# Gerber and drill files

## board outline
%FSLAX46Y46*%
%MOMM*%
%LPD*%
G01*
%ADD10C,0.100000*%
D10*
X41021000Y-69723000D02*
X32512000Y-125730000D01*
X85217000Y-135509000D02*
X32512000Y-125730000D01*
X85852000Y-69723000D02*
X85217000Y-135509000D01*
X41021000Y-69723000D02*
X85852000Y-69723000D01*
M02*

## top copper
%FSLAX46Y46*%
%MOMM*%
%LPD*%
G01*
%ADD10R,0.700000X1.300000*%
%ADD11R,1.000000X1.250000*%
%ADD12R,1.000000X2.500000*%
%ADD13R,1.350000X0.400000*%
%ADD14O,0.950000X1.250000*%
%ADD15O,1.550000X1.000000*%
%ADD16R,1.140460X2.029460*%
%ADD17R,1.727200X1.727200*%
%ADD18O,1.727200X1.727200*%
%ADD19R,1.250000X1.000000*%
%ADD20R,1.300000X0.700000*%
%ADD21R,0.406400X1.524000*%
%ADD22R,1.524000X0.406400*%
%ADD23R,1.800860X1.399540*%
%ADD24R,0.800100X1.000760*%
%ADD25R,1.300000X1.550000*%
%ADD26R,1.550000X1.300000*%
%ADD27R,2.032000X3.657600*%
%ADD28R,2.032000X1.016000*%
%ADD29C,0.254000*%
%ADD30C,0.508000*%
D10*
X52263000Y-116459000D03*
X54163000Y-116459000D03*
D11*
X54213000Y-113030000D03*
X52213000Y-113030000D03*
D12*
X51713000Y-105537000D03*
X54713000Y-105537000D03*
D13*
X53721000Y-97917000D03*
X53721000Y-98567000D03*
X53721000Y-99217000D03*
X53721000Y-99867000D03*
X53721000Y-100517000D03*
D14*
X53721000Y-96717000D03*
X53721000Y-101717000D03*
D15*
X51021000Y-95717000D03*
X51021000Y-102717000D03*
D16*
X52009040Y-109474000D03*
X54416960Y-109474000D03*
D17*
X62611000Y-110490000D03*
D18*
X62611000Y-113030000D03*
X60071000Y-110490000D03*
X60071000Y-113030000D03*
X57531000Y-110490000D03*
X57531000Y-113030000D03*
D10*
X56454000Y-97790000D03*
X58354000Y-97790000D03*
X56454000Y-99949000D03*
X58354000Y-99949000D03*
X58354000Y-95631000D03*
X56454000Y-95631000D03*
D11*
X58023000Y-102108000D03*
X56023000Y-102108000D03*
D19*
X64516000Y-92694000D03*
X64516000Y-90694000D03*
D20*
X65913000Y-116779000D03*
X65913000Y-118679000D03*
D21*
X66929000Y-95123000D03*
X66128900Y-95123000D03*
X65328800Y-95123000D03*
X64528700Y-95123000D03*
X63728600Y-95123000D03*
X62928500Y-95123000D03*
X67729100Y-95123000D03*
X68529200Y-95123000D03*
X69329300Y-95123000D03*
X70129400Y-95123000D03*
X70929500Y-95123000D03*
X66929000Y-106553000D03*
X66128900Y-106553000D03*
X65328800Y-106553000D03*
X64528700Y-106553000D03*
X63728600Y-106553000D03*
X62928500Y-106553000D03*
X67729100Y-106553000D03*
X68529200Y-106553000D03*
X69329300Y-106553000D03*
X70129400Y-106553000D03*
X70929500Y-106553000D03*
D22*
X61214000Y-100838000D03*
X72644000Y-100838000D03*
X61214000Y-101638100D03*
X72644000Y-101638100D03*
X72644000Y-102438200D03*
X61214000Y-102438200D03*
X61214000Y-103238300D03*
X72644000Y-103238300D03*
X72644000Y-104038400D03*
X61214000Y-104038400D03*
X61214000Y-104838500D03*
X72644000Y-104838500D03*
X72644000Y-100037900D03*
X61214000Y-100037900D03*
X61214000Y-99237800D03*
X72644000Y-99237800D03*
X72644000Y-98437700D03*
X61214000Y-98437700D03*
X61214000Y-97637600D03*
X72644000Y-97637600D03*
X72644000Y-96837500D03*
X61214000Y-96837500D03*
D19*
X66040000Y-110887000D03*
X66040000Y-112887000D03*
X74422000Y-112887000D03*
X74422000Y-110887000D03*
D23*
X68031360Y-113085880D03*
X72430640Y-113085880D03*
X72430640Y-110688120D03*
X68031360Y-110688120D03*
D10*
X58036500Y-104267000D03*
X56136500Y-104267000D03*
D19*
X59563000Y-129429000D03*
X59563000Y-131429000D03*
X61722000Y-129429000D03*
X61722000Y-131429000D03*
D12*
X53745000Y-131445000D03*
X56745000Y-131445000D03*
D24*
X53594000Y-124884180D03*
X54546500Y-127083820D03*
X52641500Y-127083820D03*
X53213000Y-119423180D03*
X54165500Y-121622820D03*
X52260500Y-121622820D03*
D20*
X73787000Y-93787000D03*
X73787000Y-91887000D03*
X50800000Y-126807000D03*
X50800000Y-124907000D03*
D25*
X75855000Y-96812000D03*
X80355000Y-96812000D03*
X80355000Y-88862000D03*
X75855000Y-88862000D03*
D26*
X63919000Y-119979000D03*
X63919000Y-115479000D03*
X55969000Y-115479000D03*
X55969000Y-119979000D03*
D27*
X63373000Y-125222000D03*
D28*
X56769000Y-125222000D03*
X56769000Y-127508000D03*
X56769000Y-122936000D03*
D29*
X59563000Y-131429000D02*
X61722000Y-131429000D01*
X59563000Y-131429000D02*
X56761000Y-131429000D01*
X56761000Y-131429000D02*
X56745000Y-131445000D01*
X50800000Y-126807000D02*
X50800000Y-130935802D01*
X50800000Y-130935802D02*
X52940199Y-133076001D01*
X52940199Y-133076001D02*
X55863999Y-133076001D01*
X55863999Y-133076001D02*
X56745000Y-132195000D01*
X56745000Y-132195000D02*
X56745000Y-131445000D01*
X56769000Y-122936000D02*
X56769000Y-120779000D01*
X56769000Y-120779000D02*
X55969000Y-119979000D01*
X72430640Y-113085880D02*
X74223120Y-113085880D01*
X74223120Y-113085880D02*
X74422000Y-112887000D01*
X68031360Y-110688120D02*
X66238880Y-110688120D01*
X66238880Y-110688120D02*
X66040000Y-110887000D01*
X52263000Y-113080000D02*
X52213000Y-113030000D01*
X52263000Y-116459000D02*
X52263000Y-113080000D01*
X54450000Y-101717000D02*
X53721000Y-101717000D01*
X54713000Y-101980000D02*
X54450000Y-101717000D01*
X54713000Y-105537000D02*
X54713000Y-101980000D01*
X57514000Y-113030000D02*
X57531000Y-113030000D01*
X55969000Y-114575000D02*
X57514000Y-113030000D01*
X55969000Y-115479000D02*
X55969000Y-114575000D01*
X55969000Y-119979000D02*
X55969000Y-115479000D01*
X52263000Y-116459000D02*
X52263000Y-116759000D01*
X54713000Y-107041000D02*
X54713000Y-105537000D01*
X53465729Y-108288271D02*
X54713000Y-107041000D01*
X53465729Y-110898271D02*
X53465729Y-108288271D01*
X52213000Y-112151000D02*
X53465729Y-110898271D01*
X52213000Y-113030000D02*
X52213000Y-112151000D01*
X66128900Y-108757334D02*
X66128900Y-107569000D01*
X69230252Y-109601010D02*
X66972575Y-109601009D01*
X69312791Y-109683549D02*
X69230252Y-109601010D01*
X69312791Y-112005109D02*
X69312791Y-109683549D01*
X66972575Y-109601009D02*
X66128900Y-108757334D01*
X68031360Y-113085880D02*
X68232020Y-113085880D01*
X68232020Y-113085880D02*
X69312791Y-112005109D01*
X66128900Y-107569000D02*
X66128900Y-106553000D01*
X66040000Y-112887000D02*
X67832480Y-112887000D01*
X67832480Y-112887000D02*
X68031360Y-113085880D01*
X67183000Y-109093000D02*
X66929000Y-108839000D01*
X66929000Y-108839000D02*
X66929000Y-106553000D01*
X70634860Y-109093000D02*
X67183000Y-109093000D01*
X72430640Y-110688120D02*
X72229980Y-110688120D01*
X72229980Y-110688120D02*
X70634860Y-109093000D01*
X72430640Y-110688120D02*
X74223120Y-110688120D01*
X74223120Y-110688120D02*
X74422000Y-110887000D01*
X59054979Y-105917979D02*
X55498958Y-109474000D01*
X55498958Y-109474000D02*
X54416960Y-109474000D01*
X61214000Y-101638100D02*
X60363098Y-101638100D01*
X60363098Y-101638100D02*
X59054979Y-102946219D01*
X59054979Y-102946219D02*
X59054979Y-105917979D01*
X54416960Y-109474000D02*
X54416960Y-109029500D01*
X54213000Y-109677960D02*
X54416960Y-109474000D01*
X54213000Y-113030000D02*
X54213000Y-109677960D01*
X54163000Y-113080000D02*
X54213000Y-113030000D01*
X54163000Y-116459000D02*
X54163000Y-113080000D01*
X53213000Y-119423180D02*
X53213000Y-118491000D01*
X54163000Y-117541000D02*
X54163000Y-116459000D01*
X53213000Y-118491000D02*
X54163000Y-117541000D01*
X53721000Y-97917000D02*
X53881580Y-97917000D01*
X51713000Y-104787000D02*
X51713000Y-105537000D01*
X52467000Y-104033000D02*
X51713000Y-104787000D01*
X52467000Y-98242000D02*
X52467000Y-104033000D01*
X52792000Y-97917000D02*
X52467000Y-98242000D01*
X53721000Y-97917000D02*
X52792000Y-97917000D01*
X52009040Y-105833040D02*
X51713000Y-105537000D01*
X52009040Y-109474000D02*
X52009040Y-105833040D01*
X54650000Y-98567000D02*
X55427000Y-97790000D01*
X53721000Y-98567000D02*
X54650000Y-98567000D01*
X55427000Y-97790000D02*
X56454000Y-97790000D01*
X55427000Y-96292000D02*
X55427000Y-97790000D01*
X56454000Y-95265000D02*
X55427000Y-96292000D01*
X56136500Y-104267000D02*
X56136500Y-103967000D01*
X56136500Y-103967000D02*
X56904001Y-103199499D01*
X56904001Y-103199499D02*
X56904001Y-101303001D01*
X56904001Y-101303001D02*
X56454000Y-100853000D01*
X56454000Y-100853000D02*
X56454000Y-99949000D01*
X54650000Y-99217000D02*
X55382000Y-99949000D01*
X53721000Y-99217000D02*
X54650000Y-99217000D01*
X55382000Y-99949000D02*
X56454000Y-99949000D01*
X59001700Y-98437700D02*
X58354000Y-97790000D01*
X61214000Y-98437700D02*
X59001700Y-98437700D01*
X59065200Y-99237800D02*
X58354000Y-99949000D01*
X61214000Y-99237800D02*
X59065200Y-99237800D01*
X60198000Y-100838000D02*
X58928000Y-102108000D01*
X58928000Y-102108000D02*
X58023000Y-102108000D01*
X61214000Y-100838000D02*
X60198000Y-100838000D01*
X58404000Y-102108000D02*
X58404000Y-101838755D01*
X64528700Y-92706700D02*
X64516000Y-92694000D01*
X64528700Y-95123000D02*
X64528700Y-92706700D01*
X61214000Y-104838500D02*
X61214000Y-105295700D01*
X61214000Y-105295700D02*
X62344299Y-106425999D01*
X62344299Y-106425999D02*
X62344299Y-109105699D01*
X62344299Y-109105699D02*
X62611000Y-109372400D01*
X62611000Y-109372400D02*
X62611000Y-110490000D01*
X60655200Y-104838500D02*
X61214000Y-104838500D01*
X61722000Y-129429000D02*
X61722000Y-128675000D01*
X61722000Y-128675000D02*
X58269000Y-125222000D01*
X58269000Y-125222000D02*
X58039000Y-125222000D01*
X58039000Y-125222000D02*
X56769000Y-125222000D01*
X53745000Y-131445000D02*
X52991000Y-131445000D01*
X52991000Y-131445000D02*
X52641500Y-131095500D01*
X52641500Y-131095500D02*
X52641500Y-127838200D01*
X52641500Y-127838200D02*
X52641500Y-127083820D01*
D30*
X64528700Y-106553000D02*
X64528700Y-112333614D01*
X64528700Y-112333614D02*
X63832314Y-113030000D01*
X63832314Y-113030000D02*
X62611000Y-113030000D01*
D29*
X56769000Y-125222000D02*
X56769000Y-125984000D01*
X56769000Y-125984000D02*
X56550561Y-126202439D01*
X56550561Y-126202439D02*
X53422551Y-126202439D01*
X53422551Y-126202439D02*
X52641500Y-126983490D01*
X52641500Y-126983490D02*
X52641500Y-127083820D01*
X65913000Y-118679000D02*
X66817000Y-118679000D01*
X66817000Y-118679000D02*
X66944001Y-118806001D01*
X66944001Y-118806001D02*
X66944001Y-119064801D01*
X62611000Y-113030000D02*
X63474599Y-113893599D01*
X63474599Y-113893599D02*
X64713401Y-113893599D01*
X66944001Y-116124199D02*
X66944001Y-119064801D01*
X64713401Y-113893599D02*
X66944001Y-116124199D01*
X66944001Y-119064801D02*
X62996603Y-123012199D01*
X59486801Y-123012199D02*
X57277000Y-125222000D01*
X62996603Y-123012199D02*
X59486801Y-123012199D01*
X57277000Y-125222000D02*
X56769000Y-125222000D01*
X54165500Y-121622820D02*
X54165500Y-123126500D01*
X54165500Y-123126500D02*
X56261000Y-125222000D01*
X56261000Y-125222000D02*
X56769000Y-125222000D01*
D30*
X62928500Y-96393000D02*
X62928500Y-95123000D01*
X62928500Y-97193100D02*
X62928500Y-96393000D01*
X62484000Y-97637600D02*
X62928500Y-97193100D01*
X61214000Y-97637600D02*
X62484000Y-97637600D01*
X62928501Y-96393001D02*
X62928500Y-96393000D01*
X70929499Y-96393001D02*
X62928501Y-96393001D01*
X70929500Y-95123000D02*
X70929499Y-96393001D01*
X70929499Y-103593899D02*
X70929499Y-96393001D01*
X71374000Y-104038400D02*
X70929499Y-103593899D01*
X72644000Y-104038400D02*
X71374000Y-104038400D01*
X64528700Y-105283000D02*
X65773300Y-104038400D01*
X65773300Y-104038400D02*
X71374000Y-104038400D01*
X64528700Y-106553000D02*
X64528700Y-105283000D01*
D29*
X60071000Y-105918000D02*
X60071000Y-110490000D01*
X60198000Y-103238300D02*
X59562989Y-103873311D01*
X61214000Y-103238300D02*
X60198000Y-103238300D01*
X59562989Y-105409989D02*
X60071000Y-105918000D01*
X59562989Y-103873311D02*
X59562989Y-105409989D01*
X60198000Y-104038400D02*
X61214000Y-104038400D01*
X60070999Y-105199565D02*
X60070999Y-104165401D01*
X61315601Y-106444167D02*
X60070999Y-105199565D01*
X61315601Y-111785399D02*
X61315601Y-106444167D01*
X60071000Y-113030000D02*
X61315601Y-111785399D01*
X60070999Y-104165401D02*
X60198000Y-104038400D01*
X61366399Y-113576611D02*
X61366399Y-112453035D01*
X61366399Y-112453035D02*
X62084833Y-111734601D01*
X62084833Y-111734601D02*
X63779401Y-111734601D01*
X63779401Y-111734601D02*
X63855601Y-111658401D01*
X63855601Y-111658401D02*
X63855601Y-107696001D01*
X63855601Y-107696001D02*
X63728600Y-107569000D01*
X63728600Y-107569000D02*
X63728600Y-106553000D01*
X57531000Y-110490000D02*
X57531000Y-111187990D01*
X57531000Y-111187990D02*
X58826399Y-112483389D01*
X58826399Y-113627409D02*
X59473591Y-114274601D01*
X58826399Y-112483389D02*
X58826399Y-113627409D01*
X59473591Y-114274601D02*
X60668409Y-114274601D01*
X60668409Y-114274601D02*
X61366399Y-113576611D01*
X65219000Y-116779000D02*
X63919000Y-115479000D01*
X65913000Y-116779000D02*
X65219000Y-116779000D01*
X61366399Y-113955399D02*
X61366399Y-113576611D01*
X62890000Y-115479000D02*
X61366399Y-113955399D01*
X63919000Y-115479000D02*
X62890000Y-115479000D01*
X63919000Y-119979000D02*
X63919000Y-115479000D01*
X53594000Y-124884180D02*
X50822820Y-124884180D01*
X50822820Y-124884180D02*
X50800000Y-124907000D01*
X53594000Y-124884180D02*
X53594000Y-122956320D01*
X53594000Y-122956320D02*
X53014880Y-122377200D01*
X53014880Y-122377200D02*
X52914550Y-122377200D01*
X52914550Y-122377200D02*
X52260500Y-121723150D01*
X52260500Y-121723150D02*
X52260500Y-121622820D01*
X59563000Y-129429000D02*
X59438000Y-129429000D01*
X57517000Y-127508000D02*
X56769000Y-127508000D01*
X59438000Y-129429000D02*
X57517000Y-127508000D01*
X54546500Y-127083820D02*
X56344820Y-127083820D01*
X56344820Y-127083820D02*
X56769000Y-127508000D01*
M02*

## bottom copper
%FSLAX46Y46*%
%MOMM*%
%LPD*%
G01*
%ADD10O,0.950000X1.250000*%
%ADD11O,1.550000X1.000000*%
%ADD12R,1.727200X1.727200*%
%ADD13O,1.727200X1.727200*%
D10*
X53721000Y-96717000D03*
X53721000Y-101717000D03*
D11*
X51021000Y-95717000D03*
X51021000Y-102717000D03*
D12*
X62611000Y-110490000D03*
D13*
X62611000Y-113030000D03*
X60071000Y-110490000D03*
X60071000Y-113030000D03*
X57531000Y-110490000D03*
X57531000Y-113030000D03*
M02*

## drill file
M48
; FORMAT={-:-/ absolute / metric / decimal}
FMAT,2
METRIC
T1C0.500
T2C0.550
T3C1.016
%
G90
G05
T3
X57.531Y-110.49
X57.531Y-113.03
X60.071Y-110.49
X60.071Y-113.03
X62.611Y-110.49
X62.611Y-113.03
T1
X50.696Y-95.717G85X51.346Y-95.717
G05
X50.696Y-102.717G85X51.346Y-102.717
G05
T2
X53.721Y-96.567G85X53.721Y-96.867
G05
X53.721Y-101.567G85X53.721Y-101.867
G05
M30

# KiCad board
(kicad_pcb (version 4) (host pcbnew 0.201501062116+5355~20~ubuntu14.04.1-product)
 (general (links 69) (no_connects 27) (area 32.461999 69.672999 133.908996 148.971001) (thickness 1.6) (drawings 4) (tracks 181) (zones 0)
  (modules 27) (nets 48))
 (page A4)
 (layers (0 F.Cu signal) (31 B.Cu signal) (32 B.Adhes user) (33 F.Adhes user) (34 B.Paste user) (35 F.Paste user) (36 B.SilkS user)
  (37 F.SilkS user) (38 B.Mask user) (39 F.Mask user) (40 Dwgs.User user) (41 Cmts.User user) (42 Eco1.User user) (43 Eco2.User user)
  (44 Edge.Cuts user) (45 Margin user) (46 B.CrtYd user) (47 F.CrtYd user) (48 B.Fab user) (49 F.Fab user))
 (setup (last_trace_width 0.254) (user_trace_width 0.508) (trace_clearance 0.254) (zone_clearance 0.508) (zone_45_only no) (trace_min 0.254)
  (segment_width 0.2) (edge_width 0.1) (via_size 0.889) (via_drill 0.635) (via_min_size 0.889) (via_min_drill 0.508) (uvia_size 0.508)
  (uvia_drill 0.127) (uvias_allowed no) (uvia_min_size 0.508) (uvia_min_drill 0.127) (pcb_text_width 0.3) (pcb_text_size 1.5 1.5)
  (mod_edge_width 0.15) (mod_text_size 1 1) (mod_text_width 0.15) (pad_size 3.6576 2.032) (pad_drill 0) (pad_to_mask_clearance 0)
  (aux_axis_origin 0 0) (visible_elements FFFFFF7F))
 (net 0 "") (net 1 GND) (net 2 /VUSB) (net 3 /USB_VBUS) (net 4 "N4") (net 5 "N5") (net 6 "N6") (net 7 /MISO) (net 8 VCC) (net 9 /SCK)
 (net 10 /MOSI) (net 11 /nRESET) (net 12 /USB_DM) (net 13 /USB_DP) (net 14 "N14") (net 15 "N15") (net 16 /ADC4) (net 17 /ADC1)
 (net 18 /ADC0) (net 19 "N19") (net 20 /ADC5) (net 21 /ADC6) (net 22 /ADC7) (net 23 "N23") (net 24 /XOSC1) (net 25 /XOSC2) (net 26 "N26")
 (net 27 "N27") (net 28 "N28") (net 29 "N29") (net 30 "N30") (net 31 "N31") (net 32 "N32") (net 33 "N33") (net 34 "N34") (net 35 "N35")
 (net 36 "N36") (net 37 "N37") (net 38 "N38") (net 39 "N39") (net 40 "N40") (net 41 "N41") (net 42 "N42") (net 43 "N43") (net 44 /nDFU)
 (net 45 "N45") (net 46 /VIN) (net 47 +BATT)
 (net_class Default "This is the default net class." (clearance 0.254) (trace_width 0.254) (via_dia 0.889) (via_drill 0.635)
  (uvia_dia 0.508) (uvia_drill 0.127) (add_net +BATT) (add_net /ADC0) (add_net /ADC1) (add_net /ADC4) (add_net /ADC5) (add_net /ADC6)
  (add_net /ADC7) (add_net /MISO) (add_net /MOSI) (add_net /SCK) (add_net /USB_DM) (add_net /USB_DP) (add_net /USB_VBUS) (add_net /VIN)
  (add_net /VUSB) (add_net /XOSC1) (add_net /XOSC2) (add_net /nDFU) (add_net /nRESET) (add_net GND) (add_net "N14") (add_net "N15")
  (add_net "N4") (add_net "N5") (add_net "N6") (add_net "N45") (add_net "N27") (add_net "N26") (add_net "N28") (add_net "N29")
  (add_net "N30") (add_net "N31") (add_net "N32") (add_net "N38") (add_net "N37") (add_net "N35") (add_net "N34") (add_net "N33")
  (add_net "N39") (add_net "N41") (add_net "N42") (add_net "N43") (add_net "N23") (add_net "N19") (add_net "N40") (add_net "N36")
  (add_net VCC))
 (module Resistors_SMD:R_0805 (layer F.Cu) (at 53.213 116.459)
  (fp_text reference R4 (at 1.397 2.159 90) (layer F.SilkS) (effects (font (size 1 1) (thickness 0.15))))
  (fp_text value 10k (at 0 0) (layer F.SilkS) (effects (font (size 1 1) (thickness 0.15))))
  (pad 1 smd rect (at -0.95 0) (size 0.7 1.3) (layers F.Cu F.Paste F.Mask) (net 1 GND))
  (pad 2 smd rect (at 0.95 0) (size 0.7 1.3) (layers F.Cu F.Paste F.Mask) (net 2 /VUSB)))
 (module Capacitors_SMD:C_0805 (layer F.Cu) (at 53.213 113.03 180)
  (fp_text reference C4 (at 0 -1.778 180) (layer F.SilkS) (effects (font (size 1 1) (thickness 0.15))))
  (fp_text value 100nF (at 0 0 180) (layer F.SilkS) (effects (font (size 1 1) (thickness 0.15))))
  (pad 1 smd rect (at -1 0 180) (size 1 1.25) (layers F.Cu F.Paste F.Mask) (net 2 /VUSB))
  (pad 2 smd rect (at 1 0 180) (size 1 1.25) (layers F.Cu F.Paste F.Mask) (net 1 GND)))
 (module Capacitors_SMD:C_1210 (layer F.Cu) (at 53.213 105.537)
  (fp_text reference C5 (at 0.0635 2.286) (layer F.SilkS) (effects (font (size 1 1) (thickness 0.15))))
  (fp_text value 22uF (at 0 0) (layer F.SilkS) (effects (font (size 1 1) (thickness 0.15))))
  (pad 1 smd rect (at -1.5 0) (size 1 2.5) (layers F.Cu F.Paste F.Mask) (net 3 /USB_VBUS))
  (pad 2 smd rect (at 1.5 0) (size 1 2.5) (layers F.Cu F.Paste F.Mask) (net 1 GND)))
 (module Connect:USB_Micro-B (layer F.Cu) (at 53.721 97.917)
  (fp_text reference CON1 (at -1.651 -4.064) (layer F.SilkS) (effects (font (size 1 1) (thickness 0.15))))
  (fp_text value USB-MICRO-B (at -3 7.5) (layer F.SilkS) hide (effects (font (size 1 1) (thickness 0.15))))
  (pad 1 smd rect (at 0 0) (size 1.35 0.4) (layers F.Cu F.Paste F.Mask) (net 3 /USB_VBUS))
  (pad 2 smd rect (at 0 0.65) (size 1.35 0.4) (layers F.Cu F.Paste F.Mask) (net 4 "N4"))
  (pad 3 smd rect (at 0 1.3) (size 1.35 0.4) (layers F.Cu F.Paste F.Mask) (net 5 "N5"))
  (pad 4 smd rect (at 0 1.95) (size 1.35 0.4) (layers F.Cu F.Paste F.Mask) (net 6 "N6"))
  (pad 5 smd rect (at 0 2.6) (size 1.35 0.4) (layers F.Cu F.Paste F.Mask) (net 1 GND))
  (pad 6 thru_hole oval (at 0 -1.2) (size 0.95 1.25) (drill oval 0.55 0.85) (layers *.Cu *.Mask F.SilkS) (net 1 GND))
  (pad 7 thru_hole oval (at 0 3.8) (size 0.95 1.25) (drill oval 0.55 0.85) (layers *.Cu *.Mask F.SilkS) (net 1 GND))
  (pad 8 thru_hole oval (at -2.7 -2.2) (size 1.55 1) (drill oval 1.15 0.5) (layers *.Cu *.Mask F.SilkS) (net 1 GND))
  (pad 9 thru_hole oval (at -2.7 4.8) (size 1.55 1) (drill oval 1.15 0.5) (layers *.Cu *.Mask F.SilkS) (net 1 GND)))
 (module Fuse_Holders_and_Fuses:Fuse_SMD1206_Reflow (layer F.Cu) (at 53.213 109.474)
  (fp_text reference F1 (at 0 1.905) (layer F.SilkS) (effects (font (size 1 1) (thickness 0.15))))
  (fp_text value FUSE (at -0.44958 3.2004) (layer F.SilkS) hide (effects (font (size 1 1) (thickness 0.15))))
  (pad 1 smd rect (at -1.20396 0 90) (size 2.02946 1.14046) (layers F.Cu F.Paste F.Mask) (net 3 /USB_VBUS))
  (pad 2 smd rect (at 1.20396 0 90) (size 2.02946 1.14046) (layers F.Cu F.Paste F.Mask) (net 2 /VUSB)))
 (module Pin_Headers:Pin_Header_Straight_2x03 (layer F.Cu) (at 60.071 111.76 180)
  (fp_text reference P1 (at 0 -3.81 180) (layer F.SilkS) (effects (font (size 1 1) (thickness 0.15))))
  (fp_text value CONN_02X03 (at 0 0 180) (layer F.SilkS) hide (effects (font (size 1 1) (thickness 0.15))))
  (pad 1 thru_hole rect (at -2.54 1.27 180) (size 1.7272 1.7272) (drill 1.016) (layers *.Cu *.Mask F.SilkS) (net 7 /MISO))
  (pad 2 thru_hole oval (at -2.54 -1.27 180) (size 1.7272 1.7272) (drill 1.016) (layers *.Cu *.Mask F.SilkS) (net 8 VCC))
  (pad 3 thru_hole oval (at 0 1.27 180) (size 1.7272 1.7272) (drill 1.016) (layers *.Cu *.Mask F.SilkS) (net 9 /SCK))
  (pad 4 thru_hole oval (at 0 -1.27 180) (size 1.7272 1.7272) (drill 1.016) (layers *.Cu *.Mask F.SilkS) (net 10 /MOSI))
  (pad 5 thru_hole oval (at 2.54 1.27 180) (size 1.7272 1.7272) (drill 1.016) (layers *.Cu *.Mask F.SilkS) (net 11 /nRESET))
  (pad 6 thru_hole oval (at 2.54 -1.27 180) (size 1.7272 1.7272) (drill 1.016) (layers *.Cu *.Mask F.SilkS) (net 1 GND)))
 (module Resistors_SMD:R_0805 (layer F.Cu) (at 57.404 97.79)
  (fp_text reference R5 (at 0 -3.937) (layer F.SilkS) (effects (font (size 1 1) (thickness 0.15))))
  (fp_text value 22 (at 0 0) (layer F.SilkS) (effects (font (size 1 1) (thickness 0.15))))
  (pad 1 smd rect (at -0.95 0) (size 0.7 1.3) (layers F.Cu F.Paste F.Mask) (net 4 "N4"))
  (pad 2 smd rect (at 0.95 0) (size 0.7 1.3) (layers F.Cu F.Paste F.Mask) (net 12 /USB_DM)))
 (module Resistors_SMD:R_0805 (layer F.Cu) (at 57.404 99.949)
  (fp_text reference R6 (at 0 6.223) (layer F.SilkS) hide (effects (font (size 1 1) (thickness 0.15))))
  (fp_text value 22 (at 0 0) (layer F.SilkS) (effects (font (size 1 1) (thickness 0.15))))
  (pad 1 smd rect (at -0.95 0) (size 0.7 1.3) (layers F.Cu F.Paste F.Mask) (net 5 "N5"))
  (pad 2 smd rect (at 0.95 0) (size 0.7 1.3) (layers F.Cu F.Paste F.Mask) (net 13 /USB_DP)))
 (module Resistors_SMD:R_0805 (layer F.Cu) (at 57.404 95.631 180)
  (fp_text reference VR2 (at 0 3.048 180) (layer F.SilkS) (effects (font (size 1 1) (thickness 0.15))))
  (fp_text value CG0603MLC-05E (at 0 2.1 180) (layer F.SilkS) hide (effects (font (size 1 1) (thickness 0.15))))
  (pad 1 smd rect (at -0.95 0 180) (size 0.7 1.3) (layers F.Cu F.Paste F.Mask) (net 1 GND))
  (pad 2 smd rect (at 0.95 0 180) (size 0.7 1.3) (layers F.Cu F.Paste F.Mask) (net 4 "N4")))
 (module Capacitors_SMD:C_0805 (layer F.Cu) (at 57.023 102.108 180)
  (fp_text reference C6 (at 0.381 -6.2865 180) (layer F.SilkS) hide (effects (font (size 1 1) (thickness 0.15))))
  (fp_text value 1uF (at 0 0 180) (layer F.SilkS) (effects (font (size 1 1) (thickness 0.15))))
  (pad 1 smd rect (at -1 0 180) (size 1 1.25) (layers F.Cu F.Paste F.Mask) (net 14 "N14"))
  (pad 2 smd rect (at 1 0 180) (size 1 1.25) (layers F.Cu F.Paste F.Mask) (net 1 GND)))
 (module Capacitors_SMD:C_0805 (layer F.Cu) (at 64.516 91.694 90)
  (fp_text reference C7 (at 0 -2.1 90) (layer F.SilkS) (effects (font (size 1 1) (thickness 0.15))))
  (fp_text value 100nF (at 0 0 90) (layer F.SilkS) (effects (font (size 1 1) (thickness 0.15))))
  (pad 1 smd rect (at -1 0 90) (size 1 1.25) (layers F.Cu F.Paste F.Mask) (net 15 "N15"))
  (pad 2 smd rect (at 1 0 90) (size 1 1.25) (layers F.Cu F.Paste F.Mask) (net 1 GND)))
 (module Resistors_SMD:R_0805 (layer F.Cu) (at 65.913 117.729 270)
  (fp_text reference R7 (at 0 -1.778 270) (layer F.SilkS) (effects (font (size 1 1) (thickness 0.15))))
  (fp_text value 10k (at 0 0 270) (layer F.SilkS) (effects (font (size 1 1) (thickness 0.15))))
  (pad 1 smd rect (at -0.95 0 270) (size 0.7 1.3) (layers F.Cu F.Paste F.Mask) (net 11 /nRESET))
  (pad 2 smd rect (at 0.95 0 270) (size 0.7 1.3) (layers F.Cu F.Paste F.Mask) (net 8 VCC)))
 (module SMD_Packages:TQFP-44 (layer F.Cu) (at 66.929 100.838)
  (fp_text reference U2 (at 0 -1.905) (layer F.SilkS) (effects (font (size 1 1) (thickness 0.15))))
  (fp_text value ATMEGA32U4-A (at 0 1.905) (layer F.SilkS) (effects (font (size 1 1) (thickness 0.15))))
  (pad 39 smd rect (at 0 -5.715) (size 0.4064 1.524) (layers F.Cu F.Paste F.Mask) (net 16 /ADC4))
  (pad 40 smd rect (at -0.8001 -5.715) (size 0.4064 1.524) (layers F.Cu F.Paste F.Mask) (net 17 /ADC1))
  (pad 41 smd rect (at -1.6002 -5.715) (size 0.4064 1.524) (layers F.Cu F.Paste F.Mask) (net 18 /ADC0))
  (pad 42 smd rect (at -2.4003 -5.715) (size 0.4064 1.524) (layers F.Cu F.Paste F.Mask) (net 15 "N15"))
  (pad 43 smd rect (at -3.2004 -5.715) (size 0.4064 1.524) (layers F.Cu F.Paste F.Mask) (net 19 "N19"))
  (pad 44 smd rect (at -4.0005 -5.715) (size 0.4064 1.524) (layers F.Cu F.Paste F.Mask) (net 8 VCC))
  (pad 38 smd rect (at 0.8001 -5.715) (size 0.4064 1.524) (layers F.Cu F.Paste F.Mask) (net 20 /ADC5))
  (pad 37 smd rect (at 1.6002 -5.715) (size 0.4064 1.524) (layers F.Cu F.Paste F.Mask) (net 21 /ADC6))
  (pad 36 smd rect (at 2.4003 -5.715) (size 0.4064 1.524) (layers F.Cu F.Paste F.Mask) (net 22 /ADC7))
  (pad 35 smd rect (at 3.2004 -5.715) (size 0.4064 1.524) (layers F.Cu F.Paste F.Mask) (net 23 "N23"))
  (pad 34 smd rect (at 4.0005 -5.715) (size 0.4064 1.524) (layers F.Cu F.Paste F.Mask) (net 8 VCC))
  (pad 17 smd rect (at 0 5.715) (size 0.4064 1.524) (layers F.Cu F.Paste F.Mask) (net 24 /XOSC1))
  (pad 16 smd rect (at -0.8001 5.715) (size 0.4064 1.524) (layers F.Cu F.Paste F.Mask) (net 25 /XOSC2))
  (pad 15 smd rect (at -1.6002 5.715) (size 0.4064 1.524) (layers F.Cu F.Paste F.Mask) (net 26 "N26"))
  (pad 14 smd rect (at -2.4003 5.715) (size 0.4064 1.524) (layers F.Cu F.Paste F.Mask) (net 8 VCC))
  (pad 13 smd rect (at -3.2004 5.715) (size 0.4064 1.524) (layers F.Cu F.Paste F.Mask) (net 11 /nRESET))
  (pad 12 smd rect (at -4.0005 5.715) (size 0.4064 1.524) (layers F.Cu F.Paste F.Mask) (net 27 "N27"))
  (pad 18 smd rect (at 0.8001 5.715) (size 0.4064 1.524) (layers F.Cu F.Paste F.Mask) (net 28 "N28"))
  (pad 19 smd rect (at 1.6002 5.715) (size 0.4064 1.524) (layers F.Cu F.Paste F.Mask) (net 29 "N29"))
  (pad 20 smd rect (at 2.4003 5.715) (size 0.4064 1.524) (layers F.Cu F.Paste F.Mask) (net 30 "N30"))
  (pad 21 smd rect (at 3.2004 5.715) (size 0.4064 1.524) (layers F.Cu F.Paste F.Mask) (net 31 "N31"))
  (pad 22 smd rect (at 4.0005 5.715) (size 0.4064 1.524) (layers F.Cu F.Paste F.Mask) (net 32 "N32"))
  (pad 6 smd rect (at -5.715 0) (size 1.524 0.4064) (layers F.Cu F.Paste F.Mask) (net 14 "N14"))
  (pad 28 smd rect (at 5.715 0) (size 1.524 0.4064) (layers F.Cu F.Paste F.Mask) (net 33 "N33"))
  (pad 7 smd rect (at -5.715 0.8001) (size 1.524 0.4064) (layers F.Cu F.Paste F.Mask) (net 2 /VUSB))
  (pad 27 smd rect (at 5.715 0.8001) (size 1.524 0.4064) (layers F.Cu F.Paste F.Mask) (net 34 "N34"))
  (pad 26 smd rect (at 5.715 1.6002) (size 1.524 0.4064) (layers F.Cu F.Paste F.Mask) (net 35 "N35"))
  (pad 8 smd rect (at -5.715 1.6002) (size 1.524 0.4064) (layers F.Cu F.Paste F.Mask) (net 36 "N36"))
  (pad 9 smd rect (at -5.715 2.4003) (size 1.524 0.4064) (layers F.Cu F.Paste F.Mask) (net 9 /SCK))
  (pad 25 smd rect (at 5.715 2.4003) (size 1.524 0.4064) (layers F.Cu F.Paste F.Mask) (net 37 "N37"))
  (pad 24 smd rect (at 5.715 3.2004) (size 1.524 0.4064) (layers F.Cu F.Paste F.Mask) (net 8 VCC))
  (pad 10 smd rect (at -5.715 3.2004) (size 1.524 0.4064) (layers F.Cu F.Paste F.Mask) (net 10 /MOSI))
  (pad 11 smd rect (at -5.715 4.0005) (size 1.524 0.4064) (layers F.Cu F.Paste F.Mask) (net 7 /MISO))
  (pad 23 smd rect (at 5.715 4.0005) (size 1.524 0.4064) (layers F.Cu F.Paste F.Mask) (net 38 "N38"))
  (pad 29 smd rect (at 5.715 -0.8001) (size 1.524 0.4064) (layers F.Cu F.Paste F.Mask) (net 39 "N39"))
  (pad 5 smd rect (at -5.715 -0.8001) (size 1.524 0.4064) (layers F.Cu F.Paste F.Mask) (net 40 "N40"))
  (pad 4 smd rect (at -5.715 -1.6002) (size 1.524 0.4064) (layers F.Cu F.Paste F.Mask) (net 13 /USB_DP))
  (pad 30 smd rect (at 5.715 -1.6002) (size 1.524 0.4064) (layers F.Cu F.Paste F.Mask) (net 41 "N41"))
  (pad 31 smd rect (at 5.715 -2.4003) (size 1.524 0.4064) (layers F.Cu F.Paste F.Mask) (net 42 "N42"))
  (pad 3 smd rect (at -5.715 -2.4003) (size 1.524 0.4064) (layers F.Cu F.Paste F.Mask) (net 12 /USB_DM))
  (pad 2 smd rect (at -5.715 -3.2004) (size 1.524 0.4064) (layers F.Cu F.Paste F.Mask) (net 8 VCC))
  (pad 32 smd rect (at 5.715 -3.2004) (size 1.524 0.4064) (layers F.Cu F.Paste F.Mask) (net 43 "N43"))
  (pad 33 smd rect (at 5.715 -4.0005) (size 1.524 0.4064) (layers F.Cu F.Paste F.Mask) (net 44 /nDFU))
  (pad 1 smd rect (at -5.715 -4.0005) (size 1.524 0.4064) (layers F.Cu F.Paste F.Mask) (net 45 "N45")))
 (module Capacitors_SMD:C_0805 (layer F.Cu) (at 66.04 111.887 270)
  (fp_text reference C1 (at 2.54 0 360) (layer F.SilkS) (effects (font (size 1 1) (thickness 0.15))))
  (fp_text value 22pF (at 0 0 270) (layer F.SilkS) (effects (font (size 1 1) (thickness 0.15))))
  (pad 1 smd rect (at -1 0 270) (size 1 1.25) (layers F.Cu F.Paste F.Mask) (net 1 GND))
  (pad 2 smd rect (at 1 0 270) (size 1 1.25) (layers F.Cu F.Paste F.Mask) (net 25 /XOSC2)))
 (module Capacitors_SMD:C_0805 (layer F.Cu) (at 74.422 111.887 90)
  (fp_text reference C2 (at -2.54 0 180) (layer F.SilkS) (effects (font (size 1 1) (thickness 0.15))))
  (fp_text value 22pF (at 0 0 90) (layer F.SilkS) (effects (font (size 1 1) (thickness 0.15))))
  (pad 1 smd rect (at -1 0 90) (size 1 1.25) (layers F.Cu F.Paste F.Mask) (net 1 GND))
  (pad 2 smd rect (at 1 0 90) (size 1 1.25) (layers F.Cu F.Paste F.Mask) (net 24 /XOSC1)))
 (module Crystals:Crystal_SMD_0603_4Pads (layer F.Cu) (at 70.231 111.887)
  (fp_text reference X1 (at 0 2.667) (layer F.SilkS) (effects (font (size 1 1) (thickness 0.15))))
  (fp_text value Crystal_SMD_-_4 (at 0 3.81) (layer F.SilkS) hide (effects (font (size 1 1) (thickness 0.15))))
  (pad 1 smd rect (at -2.19964 1.19888) (size 1.80086 1.39954) (layers F.Cu F.Paste F.Mask) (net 25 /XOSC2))
  (pad 2 smd rect (at 2.19964 1.19888) (size 1.80086 1.39954) (layers F.Cu F.Paste F.Mask) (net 1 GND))
  (pad 3 smd rect (at 2.19964 -1.19888) (size 1.80086 1.39954) (layers F.Cu F.Paste F.Mask) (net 24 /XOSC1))
  (pad 4 smd rect (at -2.19964 -1.19888) (size 1.80086 1.39954) (layers F.Cu F.Paste F.Mask) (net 1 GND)))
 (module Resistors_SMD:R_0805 (layer F.Cu) (at 57.0865 104.267 180)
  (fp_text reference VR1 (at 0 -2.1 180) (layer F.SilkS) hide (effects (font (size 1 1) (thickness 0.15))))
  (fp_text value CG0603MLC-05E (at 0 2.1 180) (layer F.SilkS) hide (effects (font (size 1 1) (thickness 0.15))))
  (pad 1 smd rect (at -0.95 0 180) (size 0.7 1.3) (layers F.Cu F.Paste F.Mask) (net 1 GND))
  (pad 2 smd rect (at 0.95 0 180) (size 0.7 1.3) (layers F.Cu F.Paste F.Mask) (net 5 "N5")))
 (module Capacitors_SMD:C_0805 (layer F.Cu) (at 59.563 130.429 270)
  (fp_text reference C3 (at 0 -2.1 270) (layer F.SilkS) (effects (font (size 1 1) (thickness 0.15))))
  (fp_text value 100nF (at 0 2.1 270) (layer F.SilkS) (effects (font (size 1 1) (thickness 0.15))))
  (pad 1 smd rect (at -1 0 270) (size 1 1.25) (layers F.Cu F.Paste F.Mask) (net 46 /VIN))
  (pad 2 smd rect (at 1 0 270) (size 1 1.25) (layers F.Cu F.Paste F.Mask) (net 1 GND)))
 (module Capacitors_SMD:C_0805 (layer F.Cu) (at 61.722 130.429 270)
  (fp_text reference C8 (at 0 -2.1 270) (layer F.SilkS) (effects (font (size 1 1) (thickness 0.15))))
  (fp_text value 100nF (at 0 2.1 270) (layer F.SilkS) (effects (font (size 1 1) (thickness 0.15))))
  (pad 1 smd rect (at -1 0 270) (size 1 1.25) (layers F.Cu F.Paste F.Mask) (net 8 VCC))
  (pad 2 smd rect (at 1 0 270) (size 1 1.25) (layers F.Cu F.Paste F.Mask) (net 1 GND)))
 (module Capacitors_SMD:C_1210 (layer F.Cu) (at 55.245 131.445)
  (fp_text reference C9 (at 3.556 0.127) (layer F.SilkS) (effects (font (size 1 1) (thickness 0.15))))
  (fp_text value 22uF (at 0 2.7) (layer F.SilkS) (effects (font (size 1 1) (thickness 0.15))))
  (pad 1 smd rect (at -1.5 0) (size 1 2.5) (layers F.Cu F.Paste F.Mask) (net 8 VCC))
  (pad 2 smd rect (at 1.5 0) (size 1 2.5) (layers F.Cu F.Paste F.Mask) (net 1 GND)))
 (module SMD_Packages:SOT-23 (layer F.Cu) (at 53.594 125.984)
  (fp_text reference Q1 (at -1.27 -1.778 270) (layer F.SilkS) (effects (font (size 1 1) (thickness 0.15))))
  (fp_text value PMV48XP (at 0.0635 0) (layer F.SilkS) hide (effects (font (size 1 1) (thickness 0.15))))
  (pad 3 smd rect (at 0 -1.09982) (size 0.8001 1.00076) (layers F.Cu F.Paste F.Mask) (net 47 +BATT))
  (pad 2 smd rect (at 0.9525 1.09982) (size 0.8001 1.00076) (layers F.Cu F.Paste F.Mask) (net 46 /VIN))
  (pad 1 smd rect (at -0.9525 1.09982) (size 0.8001 1.00076) (layers F.Cu F.Paste F.Mask) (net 8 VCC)))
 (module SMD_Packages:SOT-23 (layer F.Cu) (at 53.213 120.523)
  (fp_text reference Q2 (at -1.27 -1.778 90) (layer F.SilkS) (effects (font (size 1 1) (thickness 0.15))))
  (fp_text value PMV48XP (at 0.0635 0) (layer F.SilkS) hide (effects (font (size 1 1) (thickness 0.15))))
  (pad 3 smd rect (at 0 -1.09982) (size 0.8001 1.00076) (layers F.Cu F.Paste F.Mask) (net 2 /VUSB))
  (pad 2 smd rect (at 0.9525 1.09982) (size 0.8001 1.00076) (layers F.Cu F.Paste F.Mask) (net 8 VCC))
  (pad 1 smd rect (at -0.9525 1.09982) (size 0.8001 1.00076) (layers F.Cu F.Paste F.Mask) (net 47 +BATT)))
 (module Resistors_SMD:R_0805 (layer F.Cu) (at 73.787 92.837 90)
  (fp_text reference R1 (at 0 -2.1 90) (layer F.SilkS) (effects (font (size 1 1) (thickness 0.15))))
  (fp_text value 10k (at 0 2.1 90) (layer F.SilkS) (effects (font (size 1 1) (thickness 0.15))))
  (pad 1 smd rect (at -0.95 0 90) (size 0.7 1.3) (layers F.Cu F.Paste F.Mask) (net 44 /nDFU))
  (pad 2 smd rect (at 0.95 0 90) (size 0.7 1.3) (layers F.Cu F.Paste F.Mask) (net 8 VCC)))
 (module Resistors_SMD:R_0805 (layer F.Cu) (at 50.8 125.857 90)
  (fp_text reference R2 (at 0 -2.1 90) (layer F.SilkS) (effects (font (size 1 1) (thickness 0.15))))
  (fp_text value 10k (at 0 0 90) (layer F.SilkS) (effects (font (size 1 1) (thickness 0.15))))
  (pad 1 smd rect (at -0.95 0 90) (size 0.7 1.3) (layers F.Cu F.Paste F.Mask) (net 1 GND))
  (pad 2 smd rect (at 0.95 0 90) (size 0.7 1.3) (layers F.Cu F.Paste F.Mask) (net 47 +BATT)))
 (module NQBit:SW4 (layer F.Cu) (at 78.105 92.837 270)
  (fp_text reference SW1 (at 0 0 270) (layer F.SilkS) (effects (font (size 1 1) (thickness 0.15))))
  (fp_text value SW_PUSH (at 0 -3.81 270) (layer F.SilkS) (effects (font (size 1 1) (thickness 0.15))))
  (pad 2 smd rect (at 3.975 2.25 270) (size 1.55 1.3) (layers F.Cu F.Paste F.Mask) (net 44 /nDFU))
  (pad 2 smd rect (at 3.975 -2.25 270) (size 1.55 1.3) (layers F.Cu F.Paste F.Mask) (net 44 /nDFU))
  (pad 1 smd rect (at -3.975 -2.25 270) (size 1.55 1.3) (layers F.Cu F.Paste F.Mask) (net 1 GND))
  (pad 1 smd rect (at -3.975 2.25 270) (size 1.55 1.3) (layers F.Cu F.Paste F.Mask) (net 1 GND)))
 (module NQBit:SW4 (layer F.Cu) (at 59.944 117.729)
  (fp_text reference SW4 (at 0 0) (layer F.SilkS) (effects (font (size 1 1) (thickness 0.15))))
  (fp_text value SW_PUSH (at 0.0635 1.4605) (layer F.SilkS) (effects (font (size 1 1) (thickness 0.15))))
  (pad 2 smd rect (at 3.975 2.25) (size 1.55 1.3) (layers F.Cu F.Paste F.Mask) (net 11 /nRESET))
  (pad 2 smd rect (at 3.975 -2.25) (size 1.55 1.3) (layers F.Cu F.Paste F.Mask) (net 11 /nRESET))
  (pad 1 smd rect (at -3.975 -2.25) (size 1.55 1.3) (layers F.Cu F.Paste F.Mask) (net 1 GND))
  (pad 1 smd rect (at -3.975 2.25) (size 1.55 1.3) (layers F.Cu F.Paste F.Mask) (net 1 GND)))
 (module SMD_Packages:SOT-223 (layer F.Cu) (at 60.071 125.222 270)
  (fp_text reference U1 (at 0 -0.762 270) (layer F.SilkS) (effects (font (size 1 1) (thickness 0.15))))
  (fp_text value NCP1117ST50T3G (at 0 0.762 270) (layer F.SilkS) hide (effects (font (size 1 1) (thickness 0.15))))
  (pad 2 smd rect (at 0 -3.302 270) (size 3.6576 2.032) (layers F.Cu F.Paste F.Mask))
  (pad 2 smd rect (at 0 3.302 270) (size 1.016 2.032) (layers F.Cu F.Paste F.Mask) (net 8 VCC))
  (pad 3 smd rect (at 2.286 3.302 270) (size 1.016 2.032) (layers F.Cu F.Paste F.Mask) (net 46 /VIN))
  (pad 1 smd rect (at -2.286 3.302 270) (size 1.016 2.032) (layers F.Cu F.Paste F.Mask) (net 1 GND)))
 (gr_line (start 41.021 69.723) (end 32.512 125.73) (layer Edge.Cuts) (width 0.1))
 (gr_line (start 85.217 135.509) (end 32.512 125.73) (layer Edge.Cuts) (width 0.1))
 (gr_line (start 85.852 69.723) (end 85.217 135.509) (layer Edge.Cuts) (width 0.1))
 (gr_line (start 41.021 69.723) (end 85.852 69.723) (layer Edge.Cuts) (width 0.1))
 (segment (start 59.563 131.429) (end 61.722 131.429) (width 0.254) (layer F.Cu) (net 1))
 (segment (start 59.563 131.429) (end 56.761 131.429) (width 0.254) (layer F.Cu) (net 1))
 (segment (start 56.761 131.429) (end 56.745 131.445) (width 0.254) (layer F.Cu) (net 1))
 (segment (start 50.8 126.807) (end 50.8 130.935802) (width 0.254) (layer F.Cu) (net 1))
 (segment (start 50.8 130.935802) (end 52.940199 133.076001) (width 0.254) (layer F.Cu) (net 1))
 (segment (start 52.940199 133.076001) (end 55.863999 133.076001) (width 0.254) (layer F.Cu) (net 1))
 (segment (start 55.863999 133.076001) (end 56.745 132.195) (width 0.254) (layer F.Cu) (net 1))
 (segment (start 56.745 132.195) (end 56.745 131.445) (width 0.254) (layer F.Cu) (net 1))
 (segment (start 56.769 122.936) (end 56.769 120.779) (width 0.254) (layer F.Cu) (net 1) (status 10))
 (segment (start 56.769 120.779) (end 55.969 119.979) (width 0.254) (layer F.Cu) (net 1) (status 20))
 (segment (start 72.43064 113.08588) (end 74.22312 113.08588) (width 0.254) (layer F.Cu) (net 1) (status 30))
 (segment (start 74.22312 113.08588) (end 74.422 112.887) (width 0.254) (layer F.Cu) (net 1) (status 30))
 (segment (start 68.03136 110.68812) (end 66.23888 110.68812) (width 0.254) (layer F.Cu) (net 1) (status 30))
 (segment (start 66.23888 110.68812) (end 66.04 110.887) (width 0.254) (layer F.Cu) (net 1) (status 30))
 (segment (start 52.263 113.08) (end 52.213 113.03) (width 0.254) (layer F.Cu) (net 1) (status 30))
 (segment (start 52.263 116.459) (end 52.263 113.08) (width 0.254) (layer F.Cu) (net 1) (status 30))
 (segment (start 54.45 101.717) (end 53.721 101.717) (width 0.254) (layer F.Cu) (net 1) (status 20))
 (segment (start 54.713 101.98) (end 54.45 101.717) (width 0.254) (layer F.Cu) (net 1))
 (segment (start 54.713 105.537) (end 54.713 101.98) (width 0.254) (layer F.Cu) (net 1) (status 10))
 (segment (start 57.514 113.03) (end 57.531 113.03) (width 0.254) (layer F.Cu) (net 1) (status 30))
 (segment (start 55.969 114.575) (end 57.514 113.03) (width 0.254) (layer F.Cu) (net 1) (status 20))
 (segment (start 55.969 115.479) (end 55.969 114.575) (width 0.254) (layer F.Cu) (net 1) (status 10))
 (segment (start 55.969 119.979) (end 55.969 115.479) (width 0.254) (layer F.Cu) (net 1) (status 30))
 (segment (start 52.263 116.459) (end 52.263 116.759) (width 0.254) (layer F.Cu) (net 1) (status 30))
 (segment (start 54.713 107.041) (end 54.713 105.537) (width 0.254) (layer F.Cu) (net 1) (status 20))
 (segment (start 53.465729 108.288271) (end 54.713 107.041) (width 0.254) (layer F.Cu) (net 1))
 (segment (start 53.465729 110.898271) (end 53.465729 108.288271) (width 0.254) (layer F.Cu) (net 1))
 (segment (start 52.213 112.151) (end 53.465729 110.898271) (width 0.254) (layer F.Cu) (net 1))
 (segment (start 52.213 113.03) (end 52.213 112.151) (width 0.254) (layer F.Cu) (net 1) (status 10))
 (segment (start 66.1289 108.757334) (end 66.1289 107.569) (width 0.254) (layer F.Cu) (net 25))
 (segment (start 69.230252 109.60101) (end 66.972575 109.601009) (width 0.254) (layer F.Cu) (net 25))
 (segment (start 69.312791 109.683549) (end 69.230252 109.60101) (width 0.254) (layer F.Cu) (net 25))
 (segment (start 69.312791 112.005109) (end 69.312791 109.683549) (width 0.254) (layer F.Cu) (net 25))
 (segment (start 66.972575 109.601009) (end 66.1289 108.757334) (width 0.254) (layer F.Cu) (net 25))
 (segment (start 68.03136 113.08588) (end 68.23202 113.08588) (width 0.254) (layer F.Cu) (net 25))
 (segment (start 68.23202 113.08588) (end 69.312791 112.005109) (width 0.254) (layer F.Cu) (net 25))
 (segment (start 66.1289 107.569) (end 66.1289 106.553) (width 0.254) (layer F.Cu) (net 25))
 (segment (start 66.04 112.887) (end 67.83248 112.887) (width 0.254) (layer F.Cu) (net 25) (status 30))
 (segment (start 67.83248 112.887) (end 68.03136 113.08588) (width 0.254) (layer F.Cu) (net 25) (status 30))
 (segment (start 67.183 109.093) (end 66.929 108.839) (width 0.254) (layer F.Cu) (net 24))
 (segment (start 66.929 108.839) (end 66.929 106.553) (width 0.254) (layer F.Cu) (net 24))
 (segment (start 70.63486 109.093) (end 67.183 109.093) (width 0.254) (layer F.Cu) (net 24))
 (segment (start 72.43064 110.68812) (end 72.22998 110.68812) (width 0.254) (layer F.Cu) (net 24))
 (segment (start 72.22998 110.68812) (end 70.63486 109.093) (width 0.254) (layer F.Cu) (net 24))
 (segment (start 72.43064 110.68812) (end 74.22312 110.68812) (width 0.254) (layer F.Cu) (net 24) (status 30))
 (segment (start 74.22312 110.68812) (end 74.422 110.887) (width 0.254) (layer F.Cu) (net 24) (status 30))
 (segment (start 59.054979 105.917979) (end 55.498958 109.474) (width 0.254) (layer F.Cu) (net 2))
 (segment (start 55.498958 109.474) (end 54.41696 109.474) (width 0.254) (layer F.Cu) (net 2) (status 20))
 (segment (start 61.214 101.6381) (end 60.363098 101.6381) (width 0.254) (layer F.Cu) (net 2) (status 10))
 (segment (start 60.363098 101.6381) (end 59.054979 102.946219) (width 0.254) (layer F.Cu) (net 2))
 (segment (start 59.054979 102.946219) (end 59.054979 105.917979) (width 0.254) (layer F.Cu) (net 2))
 (segment (start 54.41696 109.474) (end 54.41696 109.0295) (width 0.254) (layer F.Cu) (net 2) (status 30))
 (segment (start 54.213 109.67796) (end 54.41696 109.474) (width 0.254) (layer F.Cu) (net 2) (status 30))
 (segment (start 54.213 113.03) (end 54.213 109.67796) (width 0.254) (layer F.Cu) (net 2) (status 30))
 (segment (start 54.163 113.08) (end 54.213 113.03) (width 0.254) (layer F.Cu) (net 2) (status 30))
 (segment (start 54.163 116.459) (end 54.163 113.08) (width 0.254) (layer F.Cu) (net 2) (status 30))
 (segment (start 53.213 119.42318) (end 53.213 118.491) (width 0.254) (layer F.Cu) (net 2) (status 10))
 (segment (start 54.163 117.541) (end 54.163 116.459) (width 0.254) (layer F.Cu) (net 2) (status 20))
 (segment (start 53.213 118.491) (end 54.163 117.541) (width 0.254) (layer F.Cu) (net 2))
 (segment (start 53.721 97.917) (end 53.88158 97.917) (width 0.254) (layer F.Cu) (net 3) (status 30))
 (segment (start 51.713 104.787) (end 51.713 105.537) (width 0.254) (layer F.Cu) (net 3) (status 30))
 (segment (start 52.467 104.033) (end 51.713 104.787) (width 0.254) (layer F.Cu) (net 3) (status 20))
 (segment (start 52.467 98.242) (end 52.467 104.033) (width 0.254) (layer F.Cu) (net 3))
 (segment (start 52.792 97.917) (end 52.467 98.242) (width 0.254) (layer F.Cu) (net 3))
 (segment (start 53.721 97.917) (end 52.792 97.917) (width 0.254) (layer F.Cu) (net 3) (status 10))
 (segment (start 52.00904 105.83304) (end 51.713 105.537) (width 0.254) (layer F.Cu) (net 3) (status 30))
 (segment (start 52.00904 109.474) (end 52.00904 105.83304) (width 0.254) (layer F.Cu) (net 3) (status 30))
 (segment (start 54.65 98.567) (end 55.427 97.79) (width 0.254) (layer F.Cu) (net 4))
 (segment (start 53.721 98.567) (end 54.65 98.567) (width 0.254) (layer F.Cu) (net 4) (status 10))
 (segment (start 55.427 97.79) (end 56.454 97.79) (width 0.254) (layer F.Cu) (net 4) (status 20))
 (segment (start 55.427 96.292) (end 55.427 97.79) (width 0.254) (layer F.Cu) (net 4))
 (segment (start 56.454 95.265) (end 55.427 96.292) (width 0.254) (layer F.Cu) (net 4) (status 10))
 (segment (start 56.1365 104.267) (end 56.1365 103.967) (width 0.254) (layer F.Cu) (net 5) (status 30))
 (segment (start 56.1365 103.967) (end 56.904001 103.199499) (width 0.254) (layer F.Cu) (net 5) (status 10))
 (segment (start 56.904001 103.199499) (end 56.904001 101.303001) (width 0.254) (layer F.Cu) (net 5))
 (segment (start 56.904001 101.303001) (end 56.454 100.853) (width 0.254) (layer F.Cu) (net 5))
 (segment (start 56.454 100.853) (end 56.454 99.949) (width 0.254) (layer F.Cu) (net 5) (status 20))
 (segment (start 54.65 99.217) (end 55.382 99.949) (width 0.254) (layer F.Cu) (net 5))
 (segment (start 53.721 99.217) (end 54.65 99.217) (width 0.254) (layer F.Cu) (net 5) (status 10))
 (segment (start 55.382 99.949) (end 56.454 99.949) (width 0.254) (layer F.Cu) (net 5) (status 20))
 (segment (start 59.0017 98.4377) (end 58.354 97.79) (width 0.254) (layer F.Cu) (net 12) (status 20))
 (segment (start 61.214 98.4377) (end 59.0017 98.4377) (width 0.254) (layer F.Cu) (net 12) (status 10))
 (segment (start 59.0652 99.2378) (end 58.354 99.949) (width 0.254) (layer F.Cu) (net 13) (status 20))
 (segment (start 61.214 99.2378) (end 59.0652 99.2378) (width 0.254) (layer F.Cu) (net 13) (status 10))
 (segment (start 60.198 100.838) (end 58.928 102.108) (width 0.254) (layer F.Cu) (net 14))
 (segment (start 58.928 102.108) (end 58.023 102.108) (width 0.254) (layer F.Cu) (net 14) (status 20))
 (segment (start 61.214 100.838) (end 60.198 100.838) (width 0.254) (layer F.Cu) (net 14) (status 10))
 (segment (start 58.404 102.108) (end 58.404 101.838755) (width 0.254) (layer F.Cu) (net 14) (status 30))
 (segment (start 64.5287 92.7067) (end 64.516 92.694) (width 0.254) (layer F.Cu) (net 15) (status 30))
 (segment (start 64.5287 95.123) (end 64.5287 92.7067) (width 0.254) (layer F.Cu) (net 15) (status 30))
 (segment (start 61.214 104.8385) (end 61.214 105.2957) (width 0.254) (layer F.Cu) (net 7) (status 10))
 (segment (start 61.214 105.2957) (end 62.344299 106.425999) (width 0.254) (layer F.Cu) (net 7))
 (segment (start 62.344299 106.425999) (end 62.344299 109.105699) (width 0.254) (layer F.Cu) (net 7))
 (segment (start 62.344299 109.105699) (end 62.611 109.3724) (width 0.254) (layer F.Cu) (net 7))
 (segment (start 62.611 109.3724) (end 62.611 110.49) (width 0.254) (layer F.Cu) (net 7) (status 20))
 (segment (start 60.6552 104.8385) (end 61.214 104.8385) (width 0.254) (layer F.Cu) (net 7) (status 30))
 (segment (start 61.722 129.429) (end 61.722 128.675) (width 0.254) (layer F.Cu) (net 8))
 (segment (start 61.722 128.675) (end 58.269 125.222) (width 0.254) (layer F.Cu) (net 8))
 (segment (start 58.269 125.222) (end 58.039 125.222) (width 0.254) (layer F.Cu) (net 8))
 (segment (start 58.039 125.222) (end 56.769 125.222) (width 0.254) (layer F.Cu) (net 8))
 (segment (start 53.745 131.445) (end 52.991 131.445) (width 0.254) (layer F.Cu) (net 8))
 (segment (start 52.991 131.445) (end 52.6415 131.0955) (width 0.254) (layer F.Cu) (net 8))
 (segment (start 52.6415 131.0955) (end 52.6415 127.8382) (width 0.254) (layer F.Cu) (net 8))
 (segment (start 52.6415 127.8382) (end 52.6415 127.08382) (width 0.254) (layer F.Cu) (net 8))
 (segment (start 64.5287 106.553) (end 64.5287 112.333614) (width 0.508) (layer F.Cu) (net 8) (status 10))
 (segment (start 64.5287 112.333614) (end 63.832314 113.03) (width 0.508) (layer F.Cu) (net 8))
 (segment (start 63.832314 113.03) (end 62.611 113.03) (width 0.508) (layer F.Cu) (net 8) (status 20))
 (segment (start 56.769 125.222) (end 56.769 125.984) (width 0.254) (layer F.Cu) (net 8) (status 10))
 (segment (start 56.769 125.984) (end 56.550561 126.202439) (width 0.254) (layer F.Cu) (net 8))
 (segment (start 56.550561 126.202439) (end 53.422551 126.202439) (width 0.254) (layer F.Cu) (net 8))
 (segment (start 53.422551 126.202439) (end 52.6415 126.98349) (width 0.254) (layer F.Cu) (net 8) (status 20))
 (segment (start 52.6415 126.98349) (end 52.6415 127.08382) (width 0.254) (layer F.Cu) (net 8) (status 30))
 (segment (start 65.913 118.679) (end 66.817 118.679) (width 0.254) (layer F.Cu) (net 8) (status 10))
 (segment (start 66.817 118.679) (end 66.944001 118.806001) (width 0.254) (layer F.Cu) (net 8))
 (segment (start 66.944001 118.806001) (end 66.944001 119.064801) (width 0.254) (layer F.Cu) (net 8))
 (segment (start 62.611 113.03) (end 63.474599 113.893599) (width 0.254) (layer F.Cu) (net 8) (status 10))
 (segment (start 63.474599 113.893599) (end 64.713401 113.893599) (width 0.254) (layer F.Cu) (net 8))
 (segment (start 66.944001 116.124199) (end 66.944001 119.064801) (width 0.254) (layer F.Cu) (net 8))
 (segment (start 64.713401 113.893599) (end 66.944001 116.124199) (width 0.254) (layer F.Cu) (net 8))
 (segment (start 66.944001 119.064801) (end 62.996603 123.012199) (width 0.254) (layer F.Cu) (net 8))
 (segment (start 59.486801 123.012199) (end 57.277 125.222) (width 0.254) (layer F.Cu) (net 8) (status 20))
 (segment (start 62.996603 123.012199) (end 59.486801 123.012199) (width 0.254) (layer F.Cu) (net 8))
 (segment (start 57.277 125.222) (end 56.769 125.222) (width 0.254) (layer F.Cu) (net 8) (status 30))
 (segment (start 54.1655 121.62282) (end 54.1655 123.1265) (width 0.254) (layer F.Cu) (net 8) (status 10))
 (segment (start 54.1655 123.1265) (end 56.261 125.222) (width 0.254) (layer F.Cu) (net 8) (status 20))
 (segment (start 56.261 125.222) (end 56.769 125.222) (width 0.254) (layer F.Cu) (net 8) (status 30))
 (segment (start 62.9285 96.393) (end 62.9285 95.123) (width 0.508) (layer F.Cu) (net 8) (status 20))
 (segment (start 62.9285 97.1931) (end 62.9285 96.393) (width 0.508) (layer F.Cu) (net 8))
 (segment (start 62.484 97.6376) (end 62.9285 97.1931) (width 0.508) (layer F.Cu) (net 8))
 (segment (start 61.214 97.6376) (end 62.484 97.6376) (width 0.508) (layer F.Cu) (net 8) (status 10))
 (segment (start 62.928501 96.393001) (end 62.9285 96.393) (width 0.508) (layer F.Cu) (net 8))
 (segment (start 70.929499 96.393001) (end 62.928501 96.393001) (width 0.508) (layer F.Cu) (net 8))
 (segment (start 70.9295 95.123) (end 70.929499 96.393001) (width 0.508) (layer F.Cu) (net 8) (status 10))
 (segment (start 70.929499 103.593899) (end 70.929499 96.393001) (width 0.508) (layer F.Cu) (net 8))
 (segment (start 71.374 104.0384) (end 70.929499 103.593899) (width 0.508) (layer F.Cu) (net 8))
 (segment (start 72.644 104.0384) (end 71.374 104.0384) (width 0.508) (layer F.Cu) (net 8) (status 10))
 (segment (start 64.5287 105.283) (end 65.7733 104.0384) (width 0.508) (layer F.Cu) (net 8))
 (segment (start 65.7733 104.0384) (end 71.374 104.0384) (width 0.508) (layer F.Cu) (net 8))
 (segment (start 64.5287 106.553) (end 64.5287 105.283) (width 0.508) (layer F.Cu) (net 8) (status 10))
 (segment (start 60.071 105.918) (end 60.071 110.49) (width 0.254) (layer F.Cu) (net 9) (status 20))
 (segment (start 60.198 103.2383) (end 59.562989 103.873311) (width 0.254) (layer F.Cu) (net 9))
 (segment (start 61.214 103.2383) (end 60.198 103.2383) (width 0.254) (layer F.Cu) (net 9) (status 10))
 (segment (start 59.562989 105.409989) (end 60.071 105.918) (width 0.254) (layer F.Cu) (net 9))
 (segment (start 59.562989 103.873311) (end 59.562989 105.409989) (width 0.254) (layer F.Cu) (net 9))
 (segment (start 60.198 104.0384) (end 61.214 104.0384) (width 0.254) (layer F.Cu) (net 10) (status 20))
 (segment (start 60.070999 105.199565) (end 60.070999 104.165401) (width 0.254) (layer F.Cu) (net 10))
 (segment (start 61.315601 106.444167) (end 60.070999 105.199565) (width 0.254) (layer F.Cu) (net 10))
 (segment (start 61.315601 111.785399) (end 61.315601 106.444167) (width 0.254) (layer F.Cu) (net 10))
 (segment (start 60.071 113.03) (end 61.315601 111.785399) (width 0.254) (layer F.Cu) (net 10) (status 10))
 (segment (start 60.070999 104.165401) (end 60.198 104.0384) (width 0.254) (layer F.Cu) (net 10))
 (segment (start 61.366399 113.576611) (end 61.366399 112.453035) (width 0.254) (layer F.Cu) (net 11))
 (segment (start 61.366399 112.453035) (end 62.084833 111.734601) (width 0.254) (layer F.Cu) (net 11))
 (segment (start 62.084833 111.734601) (end 63.779401 111.734601) (width 0.254) (layer F.Cu) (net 11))
 (segment (start 63.779401 111.734601) (end 63.855601 111.658401) (width 0.254) (layer F.Cu) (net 11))
 (segment (start 63.855601 111.658401) (end 63.855601 107.696001) (width 0.254) (layer F.Cu) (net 11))
 (segment (start 63.855601 107.696001) (end 63.7286 107.569) (width 0.254) (layer F.Cu) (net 11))
 (segment (start 63.7286 107.569) (end 63.7286 106.553) (width 0.254) (layer F.Cu) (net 11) (status 20))
 (segment (start 57.531 110.49) (end 57.531 111.18799) (width 0.254) (layer F.Cu) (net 11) (status 30))
 (segment (start 57.531 111.18799) (end 58.826399 112.483389) (width 0.254) (layer F.Cu) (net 11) (status 10))
 (segment (start 58.826399 113.627409) (end 59.473591 114.274601) (width 0.254) (layer F.Cu) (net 11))
 (segment (start 58.826399 112.483389) (end 58.826399 113.627409) (width 0.254) (layer F.Cu) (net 11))
 (segment (start 59.473591 114.274601) (end 60.668409 114.274601) (width 0.254) (layer F.Cu) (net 11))
 (segment (start 60.668409 114.274601) (end 61.366399 113.576611) (width 0.254) (layer F.Cu) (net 11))
 (segment (start 65.219 116.779) (end 63.919 115.479) (width 0.254) (layer F.Cu) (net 11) (status 20))
 (segment (start 65.913 116.779) (end 65.219 116.779) (width 0.254) (layer F.Cu) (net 11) (status 10))
 (segment (start 61.366399 113.955399) (end 61.366399 113.576611) (width 0.254) (layer F.Cu) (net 11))
 (segment (start 62.89 115.479) (end 61.366399 113.955399) (width 0.254) (layer F.Cu) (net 11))
 (segment (start 63.919 115.479) (end 62.89 115.479) (width 0.254) (layer F.Cu) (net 11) (status 10))
 (segment (start 63.919 119.979) (end 63.919 115.479) (width 0.254) (layer F.Cu) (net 11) (status 30))
 (segment (start 53.594 124.88418) (end 50.82282 124.88418) (width 0.254) (layer F.Cu) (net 47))
 (segment (start 50.82282 124.88418) (end 50.8 124.907) (width 0.254) (layer F.Cu) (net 47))
 (segment (start 53.594 124.88418) (end 53.594 122.95632) (width 0.254) (layer F.Cu) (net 47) (status 10))
 (segment (start 53.594 122.95632) (end 53.01488 122.3772) (width 0.254) (layer F.Cu) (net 47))
 (segment (start 53.01488 122.3772) (end 52.91455 122.3772) (width 0.254) (layer F.Cu) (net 47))
 (segment (start 52.91455 122.3772) (end 52.2605 121.72315) (width 0.254) (layer F.Cu) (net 47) (status 20))
 (segment (start 52.2605 121.72315) (end 52.2605 121.62282) (width 0.254) (layer F.Cu) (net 47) (status 30))
 (segment (start 59.563 129.429) (end 59.438 129.429) (width 0.254) (layer F.Cu) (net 46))
 (segment (start 57.517 127.508) (end 56.769 127.508) (width 0.254) (layer F.Cu) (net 46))
 (segment (start 59.438 129.429) (end 57.517 127.508) (width 0.254) (layer F.Cu) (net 46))
 (segment (start 54.5465 127.08382) (end 56.34482 127.08382) (width 0.254) (layer F.Cu) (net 46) (status 30))
 (segment (start 56.34482 127.08382) (end 56.769 127.508) (width 0.254) (layer F.Cu) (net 46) (status 30)))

